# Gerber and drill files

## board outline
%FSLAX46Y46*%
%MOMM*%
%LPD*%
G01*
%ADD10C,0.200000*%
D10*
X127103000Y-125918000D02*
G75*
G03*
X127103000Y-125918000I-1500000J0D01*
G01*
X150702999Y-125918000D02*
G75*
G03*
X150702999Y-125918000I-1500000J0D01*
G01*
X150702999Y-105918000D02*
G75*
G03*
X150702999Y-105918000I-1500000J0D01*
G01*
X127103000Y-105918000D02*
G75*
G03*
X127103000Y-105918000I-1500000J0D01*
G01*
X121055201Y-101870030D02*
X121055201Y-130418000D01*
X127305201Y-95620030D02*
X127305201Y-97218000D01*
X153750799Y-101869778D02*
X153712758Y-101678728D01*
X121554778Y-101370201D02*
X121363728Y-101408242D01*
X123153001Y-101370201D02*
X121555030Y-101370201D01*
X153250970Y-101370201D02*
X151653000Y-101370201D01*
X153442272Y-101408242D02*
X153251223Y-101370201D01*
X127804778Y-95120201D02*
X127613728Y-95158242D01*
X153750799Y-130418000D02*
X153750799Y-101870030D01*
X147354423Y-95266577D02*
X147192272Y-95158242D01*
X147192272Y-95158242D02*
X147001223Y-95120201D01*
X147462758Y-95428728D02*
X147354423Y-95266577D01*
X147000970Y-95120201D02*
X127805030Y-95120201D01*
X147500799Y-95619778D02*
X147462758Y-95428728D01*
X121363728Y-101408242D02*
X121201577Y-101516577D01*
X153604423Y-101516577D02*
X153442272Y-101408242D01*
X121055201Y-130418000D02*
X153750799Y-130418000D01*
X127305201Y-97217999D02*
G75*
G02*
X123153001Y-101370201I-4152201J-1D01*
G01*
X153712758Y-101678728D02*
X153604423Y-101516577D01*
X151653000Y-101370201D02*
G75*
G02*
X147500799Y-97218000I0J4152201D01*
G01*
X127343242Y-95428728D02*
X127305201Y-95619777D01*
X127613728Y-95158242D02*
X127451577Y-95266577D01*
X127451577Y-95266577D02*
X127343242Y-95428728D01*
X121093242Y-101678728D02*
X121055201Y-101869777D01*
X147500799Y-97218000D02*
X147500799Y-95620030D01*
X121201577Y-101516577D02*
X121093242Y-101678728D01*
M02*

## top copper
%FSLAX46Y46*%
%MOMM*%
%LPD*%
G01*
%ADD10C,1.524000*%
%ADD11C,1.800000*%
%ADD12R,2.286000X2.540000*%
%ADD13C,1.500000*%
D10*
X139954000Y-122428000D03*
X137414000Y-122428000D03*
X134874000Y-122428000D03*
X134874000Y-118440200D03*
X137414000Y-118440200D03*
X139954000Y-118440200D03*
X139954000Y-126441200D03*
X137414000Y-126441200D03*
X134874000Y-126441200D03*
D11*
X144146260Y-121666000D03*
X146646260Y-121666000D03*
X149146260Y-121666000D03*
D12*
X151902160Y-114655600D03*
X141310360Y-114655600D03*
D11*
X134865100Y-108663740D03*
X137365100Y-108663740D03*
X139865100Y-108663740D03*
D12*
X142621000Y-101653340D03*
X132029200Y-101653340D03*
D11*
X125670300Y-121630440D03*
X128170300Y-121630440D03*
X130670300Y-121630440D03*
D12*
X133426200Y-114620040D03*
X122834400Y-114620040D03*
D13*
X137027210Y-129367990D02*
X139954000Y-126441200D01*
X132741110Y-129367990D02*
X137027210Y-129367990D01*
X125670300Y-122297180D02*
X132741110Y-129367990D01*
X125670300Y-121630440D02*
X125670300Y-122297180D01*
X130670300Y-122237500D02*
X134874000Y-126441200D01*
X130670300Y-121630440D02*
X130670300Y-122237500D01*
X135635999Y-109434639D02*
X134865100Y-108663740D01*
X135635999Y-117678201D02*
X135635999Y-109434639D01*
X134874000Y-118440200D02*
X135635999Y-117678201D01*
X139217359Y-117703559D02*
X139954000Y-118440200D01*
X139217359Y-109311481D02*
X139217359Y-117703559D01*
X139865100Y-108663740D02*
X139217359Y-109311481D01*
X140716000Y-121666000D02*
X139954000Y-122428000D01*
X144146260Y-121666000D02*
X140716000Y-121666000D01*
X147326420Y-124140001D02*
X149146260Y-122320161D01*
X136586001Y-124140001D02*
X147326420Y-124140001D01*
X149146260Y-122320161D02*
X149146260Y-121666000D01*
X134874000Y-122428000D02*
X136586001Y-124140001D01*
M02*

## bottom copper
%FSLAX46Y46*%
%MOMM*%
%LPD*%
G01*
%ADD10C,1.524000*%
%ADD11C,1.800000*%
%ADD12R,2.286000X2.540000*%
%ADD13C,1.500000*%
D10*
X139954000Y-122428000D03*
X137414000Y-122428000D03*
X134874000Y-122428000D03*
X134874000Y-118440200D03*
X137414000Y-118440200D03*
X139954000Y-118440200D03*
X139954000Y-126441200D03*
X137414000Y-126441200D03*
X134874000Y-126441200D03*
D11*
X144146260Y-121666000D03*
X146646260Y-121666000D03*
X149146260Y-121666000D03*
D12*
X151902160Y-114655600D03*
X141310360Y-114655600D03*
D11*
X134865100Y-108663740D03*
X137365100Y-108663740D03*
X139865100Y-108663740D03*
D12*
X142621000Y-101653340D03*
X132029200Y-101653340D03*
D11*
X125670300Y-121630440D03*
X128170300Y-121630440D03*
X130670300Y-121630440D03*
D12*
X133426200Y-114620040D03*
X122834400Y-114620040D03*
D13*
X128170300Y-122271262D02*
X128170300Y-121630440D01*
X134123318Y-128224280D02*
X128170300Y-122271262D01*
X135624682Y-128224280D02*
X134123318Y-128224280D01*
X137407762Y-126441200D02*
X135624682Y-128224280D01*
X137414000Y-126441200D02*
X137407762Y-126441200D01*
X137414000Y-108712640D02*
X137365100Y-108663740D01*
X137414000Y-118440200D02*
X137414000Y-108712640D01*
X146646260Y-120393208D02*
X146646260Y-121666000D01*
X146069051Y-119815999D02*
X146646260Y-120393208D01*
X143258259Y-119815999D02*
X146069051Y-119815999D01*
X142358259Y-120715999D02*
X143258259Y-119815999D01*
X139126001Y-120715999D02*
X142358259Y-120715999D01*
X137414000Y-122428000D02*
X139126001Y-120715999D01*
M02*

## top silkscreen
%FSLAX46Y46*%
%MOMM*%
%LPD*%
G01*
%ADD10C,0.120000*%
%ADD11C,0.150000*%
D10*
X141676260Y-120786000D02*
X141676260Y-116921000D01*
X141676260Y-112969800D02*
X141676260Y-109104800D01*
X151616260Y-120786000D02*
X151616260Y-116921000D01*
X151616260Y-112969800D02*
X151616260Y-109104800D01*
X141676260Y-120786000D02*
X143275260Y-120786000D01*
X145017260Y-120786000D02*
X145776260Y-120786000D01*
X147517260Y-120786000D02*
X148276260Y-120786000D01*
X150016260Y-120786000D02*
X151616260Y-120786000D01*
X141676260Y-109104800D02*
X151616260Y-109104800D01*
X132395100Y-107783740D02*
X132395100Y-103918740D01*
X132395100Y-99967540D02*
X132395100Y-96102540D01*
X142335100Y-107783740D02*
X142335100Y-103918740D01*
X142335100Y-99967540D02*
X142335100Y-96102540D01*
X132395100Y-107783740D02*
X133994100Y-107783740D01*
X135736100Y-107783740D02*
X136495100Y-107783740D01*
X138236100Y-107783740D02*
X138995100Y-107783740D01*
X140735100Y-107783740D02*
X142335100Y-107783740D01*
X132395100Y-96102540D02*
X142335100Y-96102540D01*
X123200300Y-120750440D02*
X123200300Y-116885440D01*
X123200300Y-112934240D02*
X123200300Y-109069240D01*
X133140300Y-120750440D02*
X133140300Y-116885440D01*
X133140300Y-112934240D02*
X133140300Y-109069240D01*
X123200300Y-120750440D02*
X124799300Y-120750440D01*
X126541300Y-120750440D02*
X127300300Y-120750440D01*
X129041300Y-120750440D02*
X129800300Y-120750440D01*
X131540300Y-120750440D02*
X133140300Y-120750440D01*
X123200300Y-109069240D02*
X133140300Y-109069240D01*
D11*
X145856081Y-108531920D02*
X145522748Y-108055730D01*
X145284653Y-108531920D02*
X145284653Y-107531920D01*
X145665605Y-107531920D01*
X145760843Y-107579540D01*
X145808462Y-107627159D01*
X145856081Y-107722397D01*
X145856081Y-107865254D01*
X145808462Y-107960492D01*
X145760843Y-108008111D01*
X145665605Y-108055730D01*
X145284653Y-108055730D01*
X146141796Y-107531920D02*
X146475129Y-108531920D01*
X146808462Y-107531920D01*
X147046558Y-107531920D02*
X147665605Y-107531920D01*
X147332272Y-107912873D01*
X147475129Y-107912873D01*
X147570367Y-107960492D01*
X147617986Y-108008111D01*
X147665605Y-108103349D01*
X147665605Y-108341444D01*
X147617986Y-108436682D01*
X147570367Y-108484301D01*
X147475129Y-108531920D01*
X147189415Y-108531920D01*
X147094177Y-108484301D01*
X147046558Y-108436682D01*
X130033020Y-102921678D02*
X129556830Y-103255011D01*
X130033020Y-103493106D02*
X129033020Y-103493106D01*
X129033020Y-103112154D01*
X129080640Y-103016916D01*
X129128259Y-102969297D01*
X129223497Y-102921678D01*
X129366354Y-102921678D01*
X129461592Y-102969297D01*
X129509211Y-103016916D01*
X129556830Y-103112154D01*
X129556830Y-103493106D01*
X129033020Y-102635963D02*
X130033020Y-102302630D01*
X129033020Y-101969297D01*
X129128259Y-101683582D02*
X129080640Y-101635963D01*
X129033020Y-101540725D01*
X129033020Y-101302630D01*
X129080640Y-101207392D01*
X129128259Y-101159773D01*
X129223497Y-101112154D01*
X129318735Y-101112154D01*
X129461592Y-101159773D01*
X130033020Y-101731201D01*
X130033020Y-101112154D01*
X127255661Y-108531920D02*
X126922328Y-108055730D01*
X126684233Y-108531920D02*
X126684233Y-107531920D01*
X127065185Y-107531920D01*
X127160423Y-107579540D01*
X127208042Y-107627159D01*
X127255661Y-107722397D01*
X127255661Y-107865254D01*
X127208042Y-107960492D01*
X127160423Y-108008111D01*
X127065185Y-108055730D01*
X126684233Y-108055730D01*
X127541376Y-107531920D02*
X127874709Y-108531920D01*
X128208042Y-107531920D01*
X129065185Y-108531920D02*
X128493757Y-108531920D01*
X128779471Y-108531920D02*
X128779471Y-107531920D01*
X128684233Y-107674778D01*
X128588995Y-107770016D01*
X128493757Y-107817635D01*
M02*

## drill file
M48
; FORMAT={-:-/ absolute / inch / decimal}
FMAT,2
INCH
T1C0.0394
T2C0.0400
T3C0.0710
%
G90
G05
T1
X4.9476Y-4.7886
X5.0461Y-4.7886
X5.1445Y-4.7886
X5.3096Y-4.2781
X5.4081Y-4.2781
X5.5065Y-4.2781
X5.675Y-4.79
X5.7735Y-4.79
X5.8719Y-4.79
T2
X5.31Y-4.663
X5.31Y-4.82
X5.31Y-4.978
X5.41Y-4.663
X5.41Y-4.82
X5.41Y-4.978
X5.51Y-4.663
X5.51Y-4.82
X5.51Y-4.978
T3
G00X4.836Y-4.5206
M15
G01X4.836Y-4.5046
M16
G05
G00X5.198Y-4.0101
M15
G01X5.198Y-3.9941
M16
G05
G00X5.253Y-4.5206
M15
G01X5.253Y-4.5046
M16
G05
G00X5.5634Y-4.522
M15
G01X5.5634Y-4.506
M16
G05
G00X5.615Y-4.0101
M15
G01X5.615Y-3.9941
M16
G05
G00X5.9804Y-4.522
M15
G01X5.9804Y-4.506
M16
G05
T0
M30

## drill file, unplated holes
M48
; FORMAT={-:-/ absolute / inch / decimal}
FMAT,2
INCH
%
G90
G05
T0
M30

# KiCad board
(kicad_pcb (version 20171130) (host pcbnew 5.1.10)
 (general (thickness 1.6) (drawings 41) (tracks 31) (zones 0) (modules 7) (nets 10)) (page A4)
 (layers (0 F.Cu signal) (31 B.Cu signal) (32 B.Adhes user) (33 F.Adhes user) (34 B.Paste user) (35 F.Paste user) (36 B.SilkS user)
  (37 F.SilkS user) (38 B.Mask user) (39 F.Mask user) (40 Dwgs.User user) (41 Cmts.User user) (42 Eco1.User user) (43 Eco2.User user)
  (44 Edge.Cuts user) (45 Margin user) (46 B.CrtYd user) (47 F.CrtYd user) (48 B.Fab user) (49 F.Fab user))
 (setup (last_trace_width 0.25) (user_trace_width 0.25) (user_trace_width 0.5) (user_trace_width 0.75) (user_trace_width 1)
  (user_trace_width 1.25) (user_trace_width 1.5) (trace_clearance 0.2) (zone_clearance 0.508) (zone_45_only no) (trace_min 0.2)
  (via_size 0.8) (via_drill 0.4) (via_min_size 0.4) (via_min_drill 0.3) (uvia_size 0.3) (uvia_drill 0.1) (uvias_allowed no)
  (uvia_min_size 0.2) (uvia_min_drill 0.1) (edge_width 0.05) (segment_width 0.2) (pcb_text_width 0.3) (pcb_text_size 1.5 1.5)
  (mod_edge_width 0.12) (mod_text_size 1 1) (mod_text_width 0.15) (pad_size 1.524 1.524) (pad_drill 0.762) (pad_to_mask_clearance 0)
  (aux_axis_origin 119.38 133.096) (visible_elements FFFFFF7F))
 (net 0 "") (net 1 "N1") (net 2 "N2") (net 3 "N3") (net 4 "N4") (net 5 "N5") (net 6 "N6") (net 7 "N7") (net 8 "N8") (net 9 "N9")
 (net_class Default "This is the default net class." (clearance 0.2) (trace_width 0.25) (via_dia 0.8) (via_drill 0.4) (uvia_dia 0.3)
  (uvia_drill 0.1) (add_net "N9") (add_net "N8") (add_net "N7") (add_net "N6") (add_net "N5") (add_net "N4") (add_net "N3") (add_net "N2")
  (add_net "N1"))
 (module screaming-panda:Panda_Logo (layer B.Cu) (at 130.09626 106.24566 180)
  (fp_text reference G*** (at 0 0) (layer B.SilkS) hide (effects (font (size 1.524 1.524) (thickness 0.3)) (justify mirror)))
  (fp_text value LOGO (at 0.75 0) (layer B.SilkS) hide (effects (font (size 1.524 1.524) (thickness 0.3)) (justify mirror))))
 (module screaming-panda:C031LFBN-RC (layer B.Cu) (at 137.414 122.428)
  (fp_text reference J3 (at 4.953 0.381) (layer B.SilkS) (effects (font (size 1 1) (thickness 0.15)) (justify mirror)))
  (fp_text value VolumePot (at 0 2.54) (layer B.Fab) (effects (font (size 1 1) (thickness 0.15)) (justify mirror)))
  (pad 3 thru_hole circle (at 2.54 0) (size 1.524 1.524) (drill 1.016) (layers *.Cu *.Mask) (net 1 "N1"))
  (pad 2 thru_hole circle (at 0 0) (size 1.524 1.524) (drill 1.016) (layers *.Cu *.Mask) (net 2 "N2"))
  (pad 1 thru_hole circle (at -2.54 0) (size 1.524 1.524) (drill 1.016) (layers *.Cu *.Mask) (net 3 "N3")))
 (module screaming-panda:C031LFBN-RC (layer B.Cu) (at 137.414 118.4402 180)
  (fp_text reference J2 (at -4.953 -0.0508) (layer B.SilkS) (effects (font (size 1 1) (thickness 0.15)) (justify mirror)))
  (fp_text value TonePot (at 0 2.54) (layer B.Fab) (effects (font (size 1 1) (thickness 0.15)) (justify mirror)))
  (pad 3 thru_hole circle (at 2.54 0 180) (size 1.524 1.524) (drill 1.016) (layers *.Cu *.Mask) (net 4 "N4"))
  (pad 2 thru_hole circle (at 0 0 180) (size 1.524 1.524) (drill 1.016) (layers *.Cu *.Mask) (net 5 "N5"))
  (pad 1 thru_hole circle (at -2.54 0 180) (size 1.524 1.524) (drill 1.016) (layers *.Cu *.Mask) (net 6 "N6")))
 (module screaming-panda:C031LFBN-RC (layer B.Cu) (at 137.414 126.4412)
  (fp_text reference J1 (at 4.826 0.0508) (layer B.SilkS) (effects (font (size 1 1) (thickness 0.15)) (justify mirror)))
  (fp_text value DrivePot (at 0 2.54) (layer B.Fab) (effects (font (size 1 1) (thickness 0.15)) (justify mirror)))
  (pad 3 thru_hole circle (at 2.54 0) (size 1.524 1.524) (drill 1.016) (layers *.Cu *.Mask) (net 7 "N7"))
  (pad 2 thru_hole circle (at 0 0) (size 1.524 1.524) (drill 1.016) (layers *.Cu *.Mask) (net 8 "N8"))
  (pad 1 thru_hole circle (at -2.54 0) (size 1.524 1.524) (drill 1.016) (layers *.Cu *.Mask) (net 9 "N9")))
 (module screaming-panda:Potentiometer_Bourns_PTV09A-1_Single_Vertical (layer F.Cu) (at 146.60626 121.666)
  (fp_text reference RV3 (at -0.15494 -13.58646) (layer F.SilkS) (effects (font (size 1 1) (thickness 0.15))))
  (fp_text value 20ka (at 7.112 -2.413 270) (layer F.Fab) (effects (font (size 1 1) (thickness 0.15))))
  (fp_line (start -4.93 -12.5612) (end 5.01 -12.5612) (layer F.SilkS) (width 0.12))
  (fp_line (start 3.41 -0.88) (end 5.01 -0.88) (layer F.SilkS) (width 0.12))
  (fp_line (start 0.911 -0.88) (end 1.67 -0.88) (layer F.SilkS) (width 0.12))
  (fp_line (start -1.589 -0.88) (end -0.83 -0.88) (layer F.SilkS) (width 0.12))
  (fp_line (start -4.93 -0.88) (end -3.331 -0.88) (layer F.SilkS) (width 0.12))
  (fp_line (start 5.01 -8.6962) (end 5.01 -12.5612) (layer F.SilkS) (width 0.12))
  (fp_line (start 5.01 -0.88) (end 5.01 -4.745) (layer F.SilkS) (width 0.12))
  (fp_line (start -4.93 -8.6962) (end -4.93 -12.5612) (layer F.SilkS) (width 0.12))
  (fp_line (start -4.93 -0.88) (end -4.93 -4.745) (layer F.SilkS) (width 0.12))
  (pad 3 thru_hole circle (at -2.46 0 90) (size 1.8 1.8) (drill 1) (layers *.Cu *.Mask) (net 1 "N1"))
  (pad 2 thru_hole circle (at 0.04 0 90) (size 1.8 1.8) (drill 1) (layers *.Cu *.Mask) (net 2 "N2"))
  (pad 1 thru_hole circle (at 2.54 0 90) (size 1.8 1.8) (drill 1) (layers *.Cu *.Mask) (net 3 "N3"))
  (pad "" thru_hole rect (at 5.2959 -7.0104 90) (size 2.54 2.286) (drill oval 2.2098 1.8034) (layers *.Cu *.Mask))
  (pad "" thru_hole rect (at -5.2959 -7.0104 90) (size 2.54 2.286) (drill oval 2.2098 1.8034) (layers *.Cu *.Mask)))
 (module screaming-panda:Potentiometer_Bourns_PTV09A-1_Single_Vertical (layer F.Cu) (at 137.3251 108.66374)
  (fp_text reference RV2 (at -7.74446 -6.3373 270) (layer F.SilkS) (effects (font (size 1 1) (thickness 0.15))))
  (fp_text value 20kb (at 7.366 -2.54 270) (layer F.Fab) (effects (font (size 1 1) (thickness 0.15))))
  (fp_line (start -4.93 -12.5612) (end 5.01 -12.5612) (layer F.SilkS) (width 0.12))
  (fp_line (start 3.41 -0.88) (end 5.01 -0.88) (layer F.SilkS) (width 0.12))
  (fp_line (start 0.911 -0.88) (end 1.67 -0.88) (layer F.SilkS) (width 0.12))
  (fp_line (start -1.589 -0.88) (end -0.83 -0.88) (layer F.SilkS) (width 0.12))
  (fp_line (start -4.93 -0.88) (end -3.331 -0.88) (layer F.SilkS) (width 0.12))
  (fp_line (start 5.01 -8.6962) (end 5.01 -12.5612) (layer F.SilkS) (width 0.12))
  (fp_line (start 5.01 -0.88) (end 5.01 -4.745) (layer F.SilkS) (width 0.12))
  (fp_line (start -4.93 -8.6962) (end -4.93 -12.5612) (layer F.SilkS) (width 0.12))
  (fp_line (start -4.93 -0.88) (end -4.93 -4.745) (layer F.SilkS) (width 0.12))
  (pad 3 thru_hole circle (at -2.46 0 90) (size 1.8 1.8) (drill 1) (layers *.Cu *.Mask) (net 4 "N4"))
  (pad 2 thru_hole circle (at 0.04 0 90) (size 1.8 1.8) (drill 1) (layers *.Cu *.Mask) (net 5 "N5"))
  (pad 1 thru_hole circle (at 2.54 0 90) (size 1.8 1.8) (drill 1) (layers *.Cu *.Mask) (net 6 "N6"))
  (pad "" thru_hole rect (at 5.2959 -7.0104 90) (size 2.54 2.286) (drill oval 2.2098 1.8034) (layers *.Cu *.Mask))
  (pad "" thru_hole rect (at -5.2959 -7.0104 90) (size 2.54 2.286) (drill oval 2.2098 1.8034) (layers *.Cu *.Mask)))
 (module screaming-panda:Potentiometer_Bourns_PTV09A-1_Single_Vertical (layer F.Cu) (at 128.1303 121.63044)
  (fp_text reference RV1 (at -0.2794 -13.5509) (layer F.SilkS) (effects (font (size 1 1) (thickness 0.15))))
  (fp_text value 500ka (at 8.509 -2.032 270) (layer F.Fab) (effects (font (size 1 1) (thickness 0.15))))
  (fp_line (start -4.93 -12.5612) (end 5.01 -12.5612) (layer F.SilkS) (width 0.12))
  (fp_line (start 3.41 -0.88) (end 5.01 -0.88) (layer F.SilkS) (width 0.12))
  (fp_line (start 0.911 -0.88) (end 1.67 -0.88) (layer F.SilkS) (width 0.12))
  (fp_line (start -1.589 -0.88) (end -0.83 -0.88) (layer F.SilkS) (width 0.12))
  (fp_line (start -4.93 -0.88) (end -3.331 -0.88) (layer F.SilkS) (width 0.12))
  (fp_line (start 5.01 -8.6962) (end 5.01 -12.5612) (layer F.SilkS) (width 0.12))
  (fp_line (start 5.01 -0.88) (end 5.01 -4.745) (layer F.SilkS) (width 0.12))
  (fp_line (start -4.93 -8.6962) (end -4.93 -12.5612) (layer F.SilkS) (width 0.12))
  (fp_line (start -4.93 -0.88) (end -4.93 -4.745) (layer F.SilkS) (width 0.12))
  (pad 3 thru_hole circle (at -2.46 0 90) (size 1.8 1.8) (drill 1) (layers *.Cu *.Mask) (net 7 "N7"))
  (pad 2 thru_hole circle (at 0.04 0 90) (size 1.8 1.8) (drill 1) (layers *.Cu *.Mask) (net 8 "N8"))
  (pad 1 thru_hole circle (at 2.54 0 90) (size 1.8 1.8) (drill 1) (layers *.Cu *.Mask) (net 9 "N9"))
  (pad "" thru_hole rect (at 5.2959 -7.0104 90) (size 2.54 2.286) (drill oval 2.2098 1.8034) (layers *.Cu *.Mask))
  (pad "" thru_hole rect (at -5.2959 -7.0104 90) (size 2.54 2.286) (drill oval 2.2098 1.8034) (layers *.Cu *.Mask)))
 (gr_circle (center 125.603 125.918) (end 127.103 125.918) (layer Edge.Cuts) (width 0.2))
 (gr_circle (center 149.202999 125.918) (end 150.702999 125.918) (layer Edge.Cuts) (width 0.2))
 (gr_circle (center 149.202999 105.918) (end 150.702999 105.918) (layer Edge.Cuts) (width 0.2))
 (gr_circle (center 125.603 105.918) (end 127.103 105.918) (layer Edge.Cuts) (width 0.2))
 (gr_line (start 121.055201 101.87003) (end 121.055201 130.418) (layer Edge.Cuts) (width 0.2))
 (gr_line (start 127.305201 95.62003) (end 127.305201 97.218) (layer Edge.Cuts) (width 0.2))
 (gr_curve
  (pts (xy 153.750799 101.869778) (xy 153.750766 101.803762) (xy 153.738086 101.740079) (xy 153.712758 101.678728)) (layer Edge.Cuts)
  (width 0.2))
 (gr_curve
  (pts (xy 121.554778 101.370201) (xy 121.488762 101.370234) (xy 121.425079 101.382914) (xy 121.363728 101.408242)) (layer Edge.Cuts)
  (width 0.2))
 (gr_line (start 123.153001 101.370201) (end 121.55503 101.370201) (layer Edge.Cuts) (width 0.2))
 (gr_line (start 153.25097 101.370201) (end 151.653 101.370201) (layer Edge.Cuts) (width 0.2))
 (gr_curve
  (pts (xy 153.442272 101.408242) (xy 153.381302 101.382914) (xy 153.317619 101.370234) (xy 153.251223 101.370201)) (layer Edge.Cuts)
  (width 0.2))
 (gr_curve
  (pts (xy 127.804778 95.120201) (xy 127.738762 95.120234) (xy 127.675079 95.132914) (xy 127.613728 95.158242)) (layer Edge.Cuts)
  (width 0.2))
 (gr_line (start 153.750799 130.418) (end 153.750799 101.87003) (layer Edge.Cuts) (width 0.2))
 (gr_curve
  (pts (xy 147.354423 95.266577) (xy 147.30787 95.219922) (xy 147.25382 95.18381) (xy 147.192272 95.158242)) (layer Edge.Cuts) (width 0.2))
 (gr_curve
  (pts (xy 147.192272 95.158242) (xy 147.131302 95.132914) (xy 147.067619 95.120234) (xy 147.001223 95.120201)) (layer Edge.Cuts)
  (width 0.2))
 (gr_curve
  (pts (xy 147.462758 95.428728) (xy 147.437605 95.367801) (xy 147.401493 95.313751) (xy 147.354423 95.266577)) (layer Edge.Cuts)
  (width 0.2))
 (gr_line (start 147.00097 95.120201) (end 127.80503 95.120201) (layer Edge.Cuts) (width 0.2))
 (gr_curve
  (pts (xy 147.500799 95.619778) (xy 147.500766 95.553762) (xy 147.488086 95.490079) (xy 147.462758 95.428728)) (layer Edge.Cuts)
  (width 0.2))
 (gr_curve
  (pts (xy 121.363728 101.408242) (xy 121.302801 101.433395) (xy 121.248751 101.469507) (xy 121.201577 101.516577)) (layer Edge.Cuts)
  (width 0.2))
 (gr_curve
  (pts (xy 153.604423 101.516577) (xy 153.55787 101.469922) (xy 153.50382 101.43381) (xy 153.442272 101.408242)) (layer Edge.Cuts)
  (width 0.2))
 (gr_line (start 121.055201 130.418) (end 153.750799 130.418) (layer Edge.Cuts) (width 0.2))
 (gr_arc (start 123.153 97.218) (end 123.153001 101.370201) (angle -90) (layer Edge.Cuts) (width 0.2))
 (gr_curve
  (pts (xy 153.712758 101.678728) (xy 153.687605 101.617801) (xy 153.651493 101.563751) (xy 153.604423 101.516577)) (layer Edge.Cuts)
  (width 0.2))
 (gr_arc (start 151.653 97.218) (end 147.500799 97.218) (angle -90) (layer Edge.Cuts) (width 0.2))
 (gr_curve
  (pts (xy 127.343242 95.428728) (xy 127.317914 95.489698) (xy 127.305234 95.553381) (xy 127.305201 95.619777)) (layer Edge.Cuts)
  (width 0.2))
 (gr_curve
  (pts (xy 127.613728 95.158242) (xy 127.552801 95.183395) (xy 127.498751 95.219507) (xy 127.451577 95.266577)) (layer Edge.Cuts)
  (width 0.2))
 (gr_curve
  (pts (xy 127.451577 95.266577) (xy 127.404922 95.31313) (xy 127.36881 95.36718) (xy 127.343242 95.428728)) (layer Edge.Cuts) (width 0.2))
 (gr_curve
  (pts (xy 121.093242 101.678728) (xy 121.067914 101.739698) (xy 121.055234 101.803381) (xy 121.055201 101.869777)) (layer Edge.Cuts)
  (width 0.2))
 (gr_line (start 147.500799 97.218) (end 147.500799 95.62003) (layer Edge.Cuts) (width 0.2))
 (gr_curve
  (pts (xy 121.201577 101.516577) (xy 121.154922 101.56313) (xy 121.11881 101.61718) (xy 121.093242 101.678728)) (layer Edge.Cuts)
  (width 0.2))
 (segment (start 137.02721 129.36799) (end 139.954 126.4412) (width 1.5) (layer F.Cu) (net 7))
 (segment (start 132.74111 129.36799) (end 137.02721 129.36799) (width 1.5) (layer F.Cu) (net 7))
 (segment (start 125.6703 122.29718) (end 132.74111 129.36799) (width 1.5) (layer F.Cu) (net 7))
 (segment (start 125.6703 121.63044) (end 125.6703 122.29718) (width 1.5) (layer F.Cu) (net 7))
 (segment (start 128.1703 122.271262) (end 128.1703 121.63044) (width 1.5) (layer B.Cu) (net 8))
 (segment (start 134.123318 128.22428) (end 128.1703 122.271262) (width 1.5) (layer B.Cu) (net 8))
 (segment (start 135.624682 128.22428) (end 134.123318 128.22428) (width 1.5) (layer B.Cu) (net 8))
 (segment (start 137.407762 126.4412) (end 135.624682 128.22428) (width 1.5) (layer B.Cu) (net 8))
 (segment (start 137.414 126.4412) (end 137.407762 126.4412) (width 1.5) (layer B.Cu) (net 8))
 (segment (start 130.6703 122.2375) (end 134.874 126.4412) (width 1.5) (layer F.Cu) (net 9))
 (segment (start 130.6703 121.63044) (end 130.6703 122.2375) (width 1.5) (layer F.Cu) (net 9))
 (segment (start 135.635999 109.434639) (end 134.8651 108.66374) (width 1.5) (layer F.Cu) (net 4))
 (segment (start 135.635999 117.678201) (end 135.635999 109.434639) (width 1.5) (layer F.Cu) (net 4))
 (segment (start 134.874 118.4402) (end 135.635999 117.678201) (width 1.5) (layer F.Cu) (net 4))
 (segment (start 137.414 108.71264) (end 137.3651 108.66374) (width 1.5) (layer B.Cu) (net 5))
 (segment (start 137.414 118.4402) (end 137.414 108.71264) (width 1.5) (layer B.Cu) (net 5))
 (segment (start 139.217359 117.703559) (end 139.954 118.4402) (width 1.5) (layer F.Cu) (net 6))
 (segment (start 139.217359 109.311481) (end 139.217359 117.703559) (width 1.5) (layer F.Cu) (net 6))
 (segment (start 139.8651 108.66374) (end 139.217359 109.311481) (width 1.5) (layer F.Cu) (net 6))
 (segment (start 140.716 121.666) (end 139.954 122.428) (width 1.5) (layer F.Cu) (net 1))
 (segment (start 144.14626 121.666) (end 140.716 121.666) (width 1.5) (layer F.Cu) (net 1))
 (segment (start 146.64626 120.393208) (end 146.64626 121.666) (width 1.5) (layer B.Cu) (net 2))
 (segment (start 146.069051 119.815999) (end 146.64626 120.393208) (width 1.5) (layer B.Cu) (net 2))
 (segment (start 143.258259 119.815999) (end 146.069051 119.815999) (width 1.5) (layer B.Cu) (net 2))
 (segment (start 142.358259 120.715999) (end 143.258259 119.815999) (width 1.5) (layer B.Cu) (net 2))
 (segment (start 139.126001 120.715999) (end 142.358259 120.715999) (width 1.5) (layer B.Cu) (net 2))
 (segment (start 137.414 122.428) (end 139.126001 120.715999) (width 1.5) (layer B.Cu) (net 2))
 (segment (start 147.32642 124.140001) (end 149.14626 122.320161) (width 1.5) (layer F.Cu) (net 3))
 (segment (start 136.586001 124.140001) (end 147.32642 124.140001) (width 1.5) (layer F.Cu) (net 3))
 (segment (start 149.14626 122.320161) (end 149.14626 121.666) (width 1.5) (layer F.Cu) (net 3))
 (segment (start 134.874 122.428) (end 136.586001 124.140001) (width 1.5) (layer F.Cu) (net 3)))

